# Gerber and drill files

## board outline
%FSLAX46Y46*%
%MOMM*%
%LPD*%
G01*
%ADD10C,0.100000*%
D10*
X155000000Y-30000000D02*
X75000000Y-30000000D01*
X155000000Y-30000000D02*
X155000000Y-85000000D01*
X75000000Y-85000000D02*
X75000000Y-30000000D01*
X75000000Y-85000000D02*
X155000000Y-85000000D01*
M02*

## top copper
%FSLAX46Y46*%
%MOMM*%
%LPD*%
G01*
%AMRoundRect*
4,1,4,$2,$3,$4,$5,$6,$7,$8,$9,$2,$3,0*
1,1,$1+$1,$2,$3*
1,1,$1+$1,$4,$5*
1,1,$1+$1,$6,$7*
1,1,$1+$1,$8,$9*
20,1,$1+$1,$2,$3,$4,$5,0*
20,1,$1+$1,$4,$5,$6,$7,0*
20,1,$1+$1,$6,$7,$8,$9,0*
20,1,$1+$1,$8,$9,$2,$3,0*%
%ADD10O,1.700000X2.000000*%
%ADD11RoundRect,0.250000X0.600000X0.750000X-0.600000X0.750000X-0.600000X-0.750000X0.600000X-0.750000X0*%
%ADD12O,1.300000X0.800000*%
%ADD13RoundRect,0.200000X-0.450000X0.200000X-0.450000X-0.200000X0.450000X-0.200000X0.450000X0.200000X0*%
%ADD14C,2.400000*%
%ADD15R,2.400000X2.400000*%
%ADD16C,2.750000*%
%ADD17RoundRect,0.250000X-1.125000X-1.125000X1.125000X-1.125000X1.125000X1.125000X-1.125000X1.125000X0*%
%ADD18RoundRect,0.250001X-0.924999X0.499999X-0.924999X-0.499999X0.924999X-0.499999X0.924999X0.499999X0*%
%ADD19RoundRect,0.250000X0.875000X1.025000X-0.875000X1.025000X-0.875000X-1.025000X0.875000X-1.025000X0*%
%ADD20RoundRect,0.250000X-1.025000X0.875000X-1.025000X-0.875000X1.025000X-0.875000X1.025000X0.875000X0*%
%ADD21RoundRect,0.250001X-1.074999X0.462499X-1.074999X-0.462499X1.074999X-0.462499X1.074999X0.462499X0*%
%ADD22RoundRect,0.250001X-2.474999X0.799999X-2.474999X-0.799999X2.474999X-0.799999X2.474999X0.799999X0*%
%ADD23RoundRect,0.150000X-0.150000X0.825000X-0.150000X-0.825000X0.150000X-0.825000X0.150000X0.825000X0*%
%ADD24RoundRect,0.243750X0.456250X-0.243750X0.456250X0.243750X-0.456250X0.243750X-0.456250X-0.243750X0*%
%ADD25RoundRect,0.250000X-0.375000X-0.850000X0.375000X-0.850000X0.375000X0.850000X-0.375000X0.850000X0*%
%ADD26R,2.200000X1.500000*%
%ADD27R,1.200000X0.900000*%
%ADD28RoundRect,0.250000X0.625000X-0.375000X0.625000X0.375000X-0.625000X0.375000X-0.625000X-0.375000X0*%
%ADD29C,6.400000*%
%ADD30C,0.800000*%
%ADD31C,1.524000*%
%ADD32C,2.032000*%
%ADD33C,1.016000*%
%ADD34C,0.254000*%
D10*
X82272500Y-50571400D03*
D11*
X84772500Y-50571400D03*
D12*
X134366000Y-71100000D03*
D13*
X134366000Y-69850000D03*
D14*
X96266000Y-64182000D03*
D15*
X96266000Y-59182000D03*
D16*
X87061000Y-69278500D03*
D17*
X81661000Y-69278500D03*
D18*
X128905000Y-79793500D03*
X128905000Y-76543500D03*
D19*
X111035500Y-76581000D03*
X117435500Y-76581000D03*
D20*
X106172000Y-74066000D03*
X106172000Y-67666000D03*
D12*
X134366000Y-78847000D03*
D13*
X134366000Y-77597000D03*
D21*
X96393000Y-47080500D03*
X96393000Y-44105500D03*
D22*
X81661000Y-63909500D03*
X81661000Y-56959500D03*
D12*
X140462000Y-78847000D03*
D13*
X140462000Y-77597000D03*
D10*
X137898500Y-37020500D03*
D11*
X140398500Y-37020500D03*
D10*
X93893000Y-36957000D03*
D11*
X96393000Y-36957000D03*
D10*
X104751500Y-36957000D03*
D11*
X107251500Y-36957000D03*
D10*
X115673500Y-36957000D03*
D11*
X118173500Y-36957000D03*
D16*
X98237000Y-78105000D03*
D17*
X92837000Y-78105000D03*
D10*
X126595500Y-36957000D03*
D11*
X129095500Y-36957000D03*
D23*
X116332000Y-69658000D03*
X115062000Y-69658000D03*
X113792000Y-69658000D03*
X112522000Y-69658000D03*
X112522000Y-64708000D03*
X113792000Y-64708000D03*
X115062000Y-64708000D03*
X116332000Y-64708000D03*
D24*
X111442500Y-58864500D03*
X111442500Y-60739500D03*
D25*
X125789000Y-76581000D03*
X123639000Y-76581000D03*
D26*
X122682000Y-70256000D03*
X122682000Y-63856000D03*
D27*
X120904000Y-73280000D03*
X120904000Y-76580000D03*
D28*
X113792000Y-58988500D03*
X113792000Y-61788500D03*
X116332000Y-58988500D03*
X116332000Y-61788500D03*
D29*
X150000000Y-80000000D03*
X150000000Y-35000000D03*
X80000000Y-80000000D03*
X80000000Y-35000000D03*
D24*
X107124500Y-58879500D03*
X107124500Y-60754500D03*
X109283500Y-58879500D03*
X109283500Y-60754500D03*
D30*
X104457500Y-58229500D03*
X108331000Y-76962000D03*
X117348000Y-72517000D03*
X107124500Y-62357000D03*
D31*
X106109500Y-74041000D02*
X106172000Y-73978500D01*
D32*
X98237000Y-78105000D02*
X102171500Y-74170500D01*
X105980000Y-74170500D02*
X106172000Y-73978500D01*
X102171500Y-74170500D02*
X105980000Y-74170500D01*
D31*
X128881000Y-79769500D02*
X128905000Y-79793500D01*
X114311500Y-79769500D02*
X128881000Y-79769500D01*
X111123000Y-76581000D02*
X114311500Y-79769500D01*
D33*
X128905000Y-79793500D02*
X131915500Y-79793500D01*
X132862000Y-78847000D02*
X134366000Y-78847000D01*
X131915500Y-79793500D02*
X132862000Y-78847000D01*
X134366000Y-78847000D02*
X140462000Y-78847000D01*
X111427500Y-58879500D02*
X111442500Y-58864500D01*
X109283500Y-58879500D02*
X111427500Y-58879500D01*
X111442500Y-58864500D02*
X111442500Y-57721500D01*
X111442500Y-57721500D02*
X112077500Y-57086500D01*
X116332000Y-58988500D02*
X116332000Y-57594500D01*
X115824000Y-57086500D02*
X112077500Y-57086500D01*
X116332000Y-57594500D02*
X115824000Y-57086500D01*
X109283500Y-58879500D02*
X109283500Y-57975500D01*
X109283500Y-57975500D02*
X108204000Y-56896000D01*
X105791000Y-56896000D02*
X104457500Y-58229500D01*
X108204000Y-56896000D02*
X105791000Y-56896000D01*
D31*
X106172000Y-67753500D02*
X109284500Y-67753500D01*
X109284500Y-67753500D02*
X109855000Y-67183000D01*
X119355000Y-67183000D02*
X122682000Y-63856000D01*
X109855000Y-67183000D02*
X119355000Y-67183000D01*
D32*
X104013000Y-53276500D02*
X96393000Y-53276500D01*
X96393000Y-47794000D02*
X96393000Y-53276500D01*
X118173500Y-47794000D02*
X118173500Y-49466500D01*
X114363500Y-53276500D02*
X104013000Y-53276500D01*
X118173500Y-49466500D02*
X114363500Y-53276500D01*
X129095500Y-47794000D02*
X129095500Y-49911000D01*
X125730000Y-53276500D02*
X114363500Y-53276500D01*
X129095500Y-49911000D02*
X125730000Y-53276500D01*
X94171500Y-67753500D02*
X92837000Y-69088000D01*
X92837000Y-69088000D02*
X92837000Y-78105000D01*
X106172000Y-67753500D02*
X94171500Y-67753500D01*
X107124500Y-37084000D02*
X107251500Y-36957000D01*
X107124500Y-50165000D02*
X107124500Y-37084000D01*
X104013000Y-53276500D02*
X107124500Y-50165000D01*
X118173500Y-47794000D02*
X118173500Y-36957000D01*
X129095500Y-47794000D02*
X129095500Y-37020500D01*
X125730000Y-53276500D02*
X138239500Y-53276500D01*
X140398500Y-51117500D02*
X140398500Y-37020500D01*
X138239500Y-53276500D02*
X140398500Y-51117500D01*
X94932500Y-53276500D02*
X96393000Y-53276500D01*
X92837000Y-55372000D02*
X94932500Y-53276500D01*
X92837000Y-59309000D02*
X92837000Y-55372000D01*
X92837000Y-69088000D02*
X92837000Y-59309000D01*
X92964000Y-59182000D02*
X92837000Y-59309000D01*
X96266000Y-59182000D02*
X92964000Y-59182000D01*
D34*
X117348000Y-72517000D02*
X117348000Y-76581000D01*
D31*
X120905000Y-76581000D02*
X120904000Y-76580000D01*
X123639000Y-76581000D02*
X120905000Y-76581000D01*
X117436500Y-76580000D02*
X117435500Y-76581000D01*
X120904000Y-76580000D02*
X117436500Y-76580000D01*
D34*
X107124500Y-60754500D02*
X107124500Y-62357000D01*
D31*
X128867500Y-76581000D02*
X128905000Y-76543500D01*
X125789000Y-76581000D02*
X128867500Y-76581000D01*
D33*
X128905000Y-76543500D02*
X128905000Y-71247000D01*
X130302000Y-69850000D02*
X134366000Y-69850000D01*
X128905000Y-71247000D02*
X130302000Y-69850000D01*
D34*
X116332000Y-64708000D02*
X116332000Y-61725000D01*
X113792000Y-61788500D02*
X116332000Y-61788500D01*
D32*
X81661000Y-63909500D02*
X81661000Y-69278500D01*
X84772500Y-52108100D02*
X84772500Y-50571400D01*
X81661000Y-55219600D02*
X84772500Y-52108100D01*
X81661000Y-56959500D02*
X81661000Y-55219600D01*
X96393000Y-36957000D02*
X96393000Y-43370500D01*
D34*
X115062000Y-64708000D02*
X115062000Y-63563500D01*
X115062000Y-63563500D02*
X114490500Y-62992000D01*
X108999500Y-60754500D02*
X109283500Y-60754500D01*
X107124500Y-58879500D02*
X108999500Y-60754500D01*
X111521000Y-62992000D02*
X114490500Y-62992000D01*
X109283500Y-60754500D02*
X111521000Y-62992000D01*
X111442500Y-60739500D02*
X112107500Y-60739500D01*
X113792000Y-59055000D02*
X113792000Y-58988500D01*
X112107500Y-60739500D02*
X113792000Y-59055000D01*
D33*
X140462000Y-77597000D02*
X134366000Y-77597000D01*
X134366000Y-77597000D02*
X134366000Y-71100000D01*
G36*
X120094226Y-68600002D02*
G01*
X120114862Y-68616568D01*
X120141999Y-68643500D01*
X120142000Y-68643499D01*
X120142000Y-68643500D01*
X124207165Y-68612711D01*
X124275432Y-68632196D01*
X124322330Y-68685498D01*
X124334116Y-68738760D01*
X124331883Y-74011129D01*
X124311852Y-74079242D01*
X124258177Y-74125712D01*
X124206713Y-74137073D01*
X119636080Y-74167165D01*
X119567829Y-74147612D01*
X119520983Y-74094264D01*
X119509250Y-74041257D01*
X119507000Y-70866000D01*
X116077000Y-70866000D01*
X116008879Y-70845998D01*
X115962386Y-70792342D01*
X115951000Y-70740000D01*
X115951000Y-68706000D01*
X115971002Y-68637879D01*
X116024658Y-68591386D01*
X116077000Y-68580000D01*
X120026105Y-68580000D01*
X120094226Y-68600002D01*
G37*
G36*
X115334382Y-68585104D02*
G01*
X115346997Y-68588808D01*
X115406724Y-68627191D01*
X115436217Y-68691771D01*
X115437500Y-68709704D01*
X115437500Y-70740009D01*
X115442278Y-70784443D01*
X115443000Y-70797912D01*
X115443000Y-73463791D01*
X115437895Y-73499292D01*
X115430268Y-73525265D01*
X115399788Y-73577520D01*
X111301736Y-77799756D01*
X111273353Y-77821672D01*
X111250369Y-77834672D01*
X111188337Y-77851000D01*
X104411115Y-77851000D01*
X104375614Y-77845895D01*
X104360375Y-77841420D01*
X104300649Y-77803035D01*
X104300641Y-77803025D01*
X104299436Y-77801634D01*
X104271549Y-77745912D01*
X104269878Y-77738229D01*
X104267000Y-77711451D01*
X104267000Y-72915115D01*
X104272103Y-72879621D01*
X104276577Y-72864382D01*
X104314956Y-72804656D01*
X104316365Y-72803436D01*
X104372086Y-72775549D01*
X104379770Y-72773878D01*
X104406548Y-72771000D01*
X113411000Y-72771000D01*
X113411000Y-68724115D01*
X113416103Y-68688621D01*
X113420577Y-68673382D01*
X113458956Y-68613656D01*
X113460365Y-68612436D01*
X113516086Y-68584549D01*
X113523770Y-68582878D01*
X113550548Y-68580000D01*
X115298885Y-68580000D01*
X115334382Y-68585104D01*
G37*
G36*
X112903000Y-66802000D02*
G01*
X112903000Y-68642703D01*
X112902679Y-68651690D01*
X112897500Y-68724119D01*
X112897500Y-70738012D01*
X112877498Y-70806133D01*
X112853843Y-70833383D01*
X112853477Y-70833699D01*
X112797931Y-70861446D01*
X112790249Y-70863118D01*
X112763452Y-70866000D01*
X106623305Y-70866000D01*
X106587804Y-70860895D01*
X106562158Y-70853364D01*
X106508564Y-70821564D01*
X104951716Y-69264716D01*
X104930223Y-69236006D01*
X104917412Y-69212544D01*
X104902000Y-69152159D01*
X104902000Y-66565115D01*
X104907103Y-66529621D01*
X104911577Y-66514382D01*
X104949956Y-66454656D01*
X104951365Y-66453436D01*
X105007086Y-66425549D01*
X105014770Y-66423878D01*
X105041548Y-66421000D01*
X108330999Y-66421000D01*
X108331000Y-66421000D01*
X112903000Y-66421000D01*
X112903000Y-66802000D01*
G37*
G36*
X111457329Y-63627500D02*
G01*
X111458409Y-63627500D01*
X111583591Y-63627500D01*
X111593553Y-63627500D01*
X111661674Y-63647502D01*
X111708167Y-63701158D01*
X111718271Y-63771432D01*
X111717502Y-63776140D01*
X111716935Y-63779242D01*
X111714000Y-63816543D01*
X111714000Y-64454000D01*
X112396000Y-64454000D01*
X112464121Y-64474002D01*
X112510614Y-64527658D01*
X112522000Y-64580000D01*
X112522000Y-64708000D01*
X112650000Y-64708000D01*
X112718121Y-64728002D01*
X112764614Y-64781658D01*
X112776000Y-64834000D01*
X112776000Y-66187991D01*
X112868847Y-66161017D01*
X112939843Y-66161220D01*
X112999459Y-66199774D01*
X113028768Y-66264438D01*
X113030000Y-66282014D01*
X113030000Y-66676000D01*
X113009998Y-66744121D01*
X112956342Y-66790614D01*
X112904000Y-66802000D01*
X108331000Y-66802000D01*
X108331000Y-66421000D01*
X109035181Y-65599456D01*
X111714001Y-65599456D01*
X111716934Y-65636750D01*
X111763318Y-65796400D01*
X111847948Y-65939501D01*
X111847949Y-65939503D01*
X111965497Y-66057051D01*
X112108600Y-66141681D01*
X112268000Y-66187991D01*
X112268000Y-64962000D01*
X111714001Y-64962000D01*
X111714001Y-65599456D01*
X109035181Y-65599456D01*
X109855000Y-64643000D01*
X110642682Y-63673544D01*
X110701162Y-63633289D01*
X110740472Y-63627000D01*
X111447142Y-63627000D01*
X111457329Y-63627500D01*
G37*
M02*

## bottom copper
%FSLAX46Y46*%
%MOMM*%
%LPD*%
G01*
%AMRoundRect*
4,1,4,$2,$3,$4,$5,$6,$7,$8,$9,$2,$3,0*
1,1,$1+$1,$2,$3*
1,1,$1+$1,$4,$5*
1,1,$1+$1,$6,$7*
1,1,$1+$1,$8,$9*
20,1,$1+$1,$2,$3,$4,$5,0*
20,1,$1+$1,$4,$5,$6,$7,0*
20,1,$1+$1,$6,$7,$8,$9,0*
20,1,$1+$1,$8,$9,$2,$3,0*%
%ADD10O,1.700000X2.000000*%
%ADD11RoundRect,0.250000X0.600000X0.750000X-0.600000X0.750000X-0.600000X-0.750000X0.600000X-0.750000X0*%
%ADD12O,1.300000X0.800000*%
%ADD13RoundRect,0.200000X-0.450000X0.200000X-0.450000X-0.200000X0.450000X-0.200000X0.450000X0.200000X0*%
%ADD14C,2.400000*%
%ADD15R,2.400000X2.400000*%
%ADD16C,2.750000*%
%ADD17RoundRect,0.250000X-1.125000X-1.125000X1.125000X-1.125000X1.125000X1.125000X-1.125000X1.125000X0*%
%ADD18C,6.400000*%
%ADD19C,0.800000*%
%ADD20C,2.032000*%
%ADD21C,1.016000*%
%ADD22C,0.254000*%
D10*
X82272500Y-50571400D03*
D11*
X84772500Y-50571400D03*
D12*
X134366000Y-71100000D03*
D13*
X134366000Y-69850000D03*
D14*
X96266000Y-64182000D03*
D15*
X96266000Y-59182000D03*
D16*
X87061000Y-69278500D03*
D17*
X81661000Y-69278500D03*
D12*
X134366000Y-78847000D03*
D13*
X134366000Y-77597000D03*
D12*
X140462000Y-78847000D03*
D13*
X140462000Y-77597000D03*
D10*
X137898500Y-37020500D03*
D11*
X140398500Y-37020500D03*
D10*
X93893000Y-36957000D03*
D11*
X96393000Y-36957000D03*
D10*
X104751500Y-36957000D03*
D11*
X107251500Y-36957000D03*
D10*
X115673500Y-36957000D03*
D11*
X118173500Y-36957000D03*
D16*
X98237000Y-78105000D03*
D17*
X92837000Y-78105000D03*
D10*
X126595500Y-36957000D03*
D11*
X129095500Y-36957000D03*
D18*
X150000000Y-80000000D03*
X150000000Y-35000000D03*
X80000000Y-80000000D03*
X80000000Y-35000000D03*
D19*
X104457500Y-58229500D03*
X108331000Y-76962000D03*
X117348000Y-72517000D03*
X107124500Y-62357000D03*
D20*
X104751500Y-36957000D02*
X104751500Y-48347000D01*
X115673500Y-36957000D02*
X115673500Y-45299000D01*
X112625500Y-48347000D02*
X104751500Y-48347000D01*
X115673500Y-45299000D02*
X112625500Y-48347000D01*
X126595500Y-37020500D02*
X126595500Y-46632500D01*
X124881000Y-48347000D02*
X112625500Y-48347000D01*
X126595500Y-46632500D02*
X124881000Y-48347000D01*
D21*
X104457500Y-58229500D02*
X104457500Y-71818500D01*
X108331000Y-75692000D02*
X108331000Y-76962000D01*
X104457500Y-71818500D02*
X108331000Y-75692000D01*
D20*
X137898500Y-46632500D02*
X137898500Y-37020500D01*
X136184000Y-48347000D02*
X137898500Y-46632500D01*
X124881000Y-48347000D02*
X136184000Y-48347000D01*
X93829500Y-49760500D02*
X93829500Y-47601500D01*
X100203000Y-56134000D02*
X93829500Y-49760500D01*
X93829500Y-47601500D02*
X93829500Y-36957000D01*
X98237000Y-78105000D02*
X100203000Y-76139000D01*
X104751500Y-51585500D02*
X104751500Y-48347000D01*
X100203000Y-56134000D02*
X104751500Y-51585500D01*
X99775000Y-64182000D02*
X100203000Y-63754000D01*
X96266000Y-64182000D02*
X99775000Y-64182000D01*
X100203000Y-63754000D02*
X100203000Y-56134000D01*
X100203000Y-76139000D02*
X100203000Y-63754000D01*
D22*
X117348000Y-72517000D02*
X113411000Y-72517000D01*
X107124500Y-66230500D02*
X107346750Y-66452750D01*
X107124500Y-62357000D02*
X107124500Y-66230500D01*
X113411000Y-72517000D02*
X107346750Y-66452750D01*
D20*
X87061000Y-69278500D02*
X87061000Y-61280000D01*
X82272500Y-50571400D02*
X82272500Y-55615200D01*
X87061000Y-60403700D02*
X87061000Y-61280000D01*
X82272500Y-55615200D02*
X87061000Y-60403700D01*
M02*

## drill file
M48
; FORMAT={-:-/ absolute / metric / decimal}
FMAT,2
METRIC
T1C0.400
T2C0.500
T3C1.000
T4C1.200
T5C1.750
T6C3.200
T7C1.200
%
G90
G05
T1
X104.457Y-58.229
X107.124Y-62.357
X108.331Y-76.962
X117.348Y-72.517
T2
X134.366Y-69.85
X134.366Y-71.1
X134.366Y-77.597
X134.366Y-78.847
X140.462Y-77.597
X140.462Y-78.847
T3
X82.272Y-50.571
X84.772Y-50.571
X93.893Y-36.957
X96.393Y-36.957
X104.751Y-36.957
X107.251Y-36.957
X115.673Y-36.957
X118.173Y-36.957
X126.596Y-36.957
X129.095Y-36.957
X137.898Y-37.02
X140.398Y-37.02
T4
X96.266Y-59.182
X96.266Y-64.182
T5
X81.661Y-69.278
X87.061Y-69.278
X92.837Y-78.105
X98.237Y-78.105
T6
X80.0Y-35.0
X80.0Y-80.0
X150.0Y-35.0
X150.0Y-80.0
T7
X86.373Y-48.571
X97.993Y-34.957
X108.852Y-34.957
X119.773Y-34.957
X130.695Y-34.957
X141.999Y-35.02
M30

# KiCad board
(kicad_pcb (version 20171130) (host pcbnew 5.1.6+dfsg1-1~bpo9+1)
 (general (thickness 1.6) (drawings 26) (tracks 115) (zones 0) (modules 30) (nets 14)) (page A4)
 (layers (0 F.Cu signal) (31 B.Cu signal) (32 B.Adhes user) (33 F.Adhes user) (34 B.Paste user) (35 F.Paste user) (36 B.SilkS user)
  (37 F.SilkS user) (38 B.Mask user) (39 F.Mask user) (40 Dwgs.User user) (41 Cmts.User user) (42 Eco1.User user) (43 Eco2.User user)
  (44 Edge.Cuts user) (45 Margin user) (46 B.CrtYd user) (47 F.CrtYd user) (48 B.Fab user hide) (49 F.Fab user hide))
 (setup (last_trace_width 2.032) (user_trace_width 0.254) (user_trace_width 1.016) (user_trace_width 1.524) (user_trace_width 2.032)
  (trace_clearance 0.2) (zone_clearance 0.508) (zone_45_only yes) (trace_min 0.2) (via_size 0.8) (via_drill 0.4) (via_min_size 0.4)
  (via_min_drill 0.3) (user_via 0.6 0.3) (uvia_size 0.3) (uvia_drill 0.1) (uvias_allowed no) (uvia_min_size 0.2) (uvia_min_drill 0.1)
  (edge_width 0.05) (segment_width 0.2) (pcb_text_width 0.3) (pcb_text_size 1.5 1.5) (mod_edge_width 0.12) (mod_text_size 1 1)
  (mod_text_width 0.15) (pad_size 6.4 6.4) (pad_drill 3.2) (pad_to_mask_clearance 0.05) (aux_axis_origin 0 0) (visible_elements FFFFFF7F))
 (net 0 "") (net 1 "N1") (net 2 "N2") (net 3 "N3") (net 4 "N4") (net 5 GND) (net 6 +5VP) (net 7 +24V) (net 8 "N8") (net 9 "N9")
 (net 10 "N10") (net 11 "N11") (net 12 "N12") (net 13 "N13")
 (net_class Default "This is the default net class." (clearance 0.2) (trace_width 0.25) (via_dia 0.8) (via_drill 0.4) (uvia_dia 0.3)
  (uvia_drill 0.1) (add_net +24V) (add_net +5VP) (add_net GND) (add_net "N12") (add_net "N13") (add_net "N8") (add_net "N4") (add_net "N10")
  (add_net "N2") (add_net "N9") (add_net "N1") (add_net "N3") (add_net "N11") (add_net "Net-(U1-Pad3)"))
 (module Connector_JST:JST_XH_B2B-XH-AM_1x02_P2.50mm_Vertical (layer F.Cu) (at 84.7725 50.5714 180)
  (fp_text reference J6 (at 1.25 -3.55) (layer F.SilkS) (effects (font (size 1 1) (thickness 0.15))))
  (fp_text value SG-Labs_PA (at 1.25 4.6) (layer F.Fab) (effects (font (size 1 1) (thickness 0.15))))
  (pad "" np_thru_hole circle (at -1.6 2 180) (size 1.2 1.2) (drill 1.2) (layers *.Cu *.Mask))
  (pad 2 thru_hole oval (at 2.5 0 180) (size 1.7 2) (drill 1) (layers *.Cu *.Mask) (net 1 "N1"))
  (pad 1 thru_hole roundrect (at 0 0 180) (size 1.7 2) (drill 1) (layers *.Cu *.Mask) (roundrect_rratio 0.147059) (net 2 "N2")))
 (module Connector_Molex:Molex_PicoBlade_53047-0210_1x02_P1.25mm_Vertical (layer F.Cu) (at 134.366 69.85 270)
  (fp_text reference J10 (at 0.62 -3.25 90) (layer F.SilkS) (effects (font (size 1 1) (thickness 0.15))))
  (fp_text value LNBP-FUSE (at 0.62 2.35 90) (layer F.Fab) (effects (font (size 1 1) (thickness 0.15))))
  (pad 2 thru_hole oval (at 1.25 0 270) (size 0.8 1.3) (drill 0.5) (layers *.Cu *.Mask) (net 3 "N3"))
  (pad 1 thru_hole roundrect (at 0 0 270) (size 0.8 1.3) (drill 0.5) (layers *.Cu *.Mask) (roundrect_rratio 0.25) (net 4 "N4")))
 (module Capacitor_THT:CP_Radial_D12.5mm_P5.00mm (layer F.Cu) (at 96.266 59.182 270)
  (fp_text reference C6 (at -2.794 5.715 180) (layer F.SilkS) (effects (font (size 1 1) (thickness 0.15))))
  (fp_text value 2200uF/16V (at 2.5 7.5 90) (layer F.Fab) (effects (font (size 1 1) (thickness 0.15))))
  (pad 2 thru_hole circle (at 5 0 270) (size 2.4 2.4) (drill 1.2) (layers *.Cu *.Mask) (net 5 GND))
  (pad 1 thru_hole rect (at 0 0 270) (size 2.4 2.4) (drill 1.2) (layers *.Cu *.Mask) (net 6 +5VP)))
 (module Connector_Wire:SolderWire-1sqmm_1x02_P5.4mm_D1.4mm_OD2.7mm (layer F.Cu) (at 81.661 69.2785)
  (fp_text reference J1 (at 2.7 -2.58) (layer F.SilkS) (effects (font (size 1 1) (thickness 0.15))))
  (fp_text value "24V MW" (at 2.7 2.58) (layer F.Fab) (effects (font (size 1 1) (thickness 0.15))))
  (pad 2 thru_hole circle (at 5.4 0) (size 2.75 2.75) (drill 1.75) (layers *.Cu *.Mask) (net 1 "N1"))
  (pad 1 thru_hole roundrect (at 0 0) (size 2.75 2.75) (drill 1.75) (layers *.Cu *.Mask) (roundrect_rratio 0.090909) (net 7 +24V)))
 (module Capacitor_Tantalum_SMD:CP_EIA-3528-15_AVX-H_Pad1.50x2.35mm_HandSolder (layer F.Cu) (at 128.905 78.1685 270)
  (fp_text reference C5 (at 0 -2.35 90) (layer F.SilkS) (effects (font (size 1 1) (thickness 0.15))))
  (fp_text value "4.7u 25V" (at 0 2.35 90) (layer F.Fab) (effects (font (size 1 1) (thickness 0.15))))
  (pad 2 smd roundrect (at 1.625 0 270) (size 1.5 2.35) (layers F.Cu F.Paste F.Mask) (roundrect_rratio 0.166667) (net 5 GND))
  (pad 1 smd roundrect (at -1.625 0 270) (size 1.5 2.35) (layers F.Cu F.Paste F.Mask) (roundrect_rratio 0.166667) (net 4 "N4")))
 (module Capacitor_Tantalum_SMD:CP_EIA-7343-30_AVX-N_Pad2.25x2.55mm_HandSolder (layer F.Cu) (at 114.2355 76.581 180)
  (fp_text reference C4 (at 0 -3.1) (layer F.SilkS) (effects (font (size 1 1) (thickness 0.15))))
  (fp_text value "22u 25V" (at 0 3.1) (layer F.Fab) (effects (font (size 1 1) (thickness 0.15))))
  (pad 2 smd roundrect (at 3.2 0 180) (size 2.25 2.55) (layers F.Cu F.Paste F.Mask) (roundrect_rratio 0.111111) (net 5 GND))
  (pad 1 smd roundrect (at -3.2 0 180) (size 2.25 2.55) (layers F.Cu F.Paste F.Mask) (roundrect_rratio 0.111111) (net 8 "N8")))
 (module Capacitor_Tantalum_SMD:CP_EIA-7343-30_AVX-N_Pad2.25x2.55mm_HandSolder (layer F.Cu) (at 106.172 70.866 270)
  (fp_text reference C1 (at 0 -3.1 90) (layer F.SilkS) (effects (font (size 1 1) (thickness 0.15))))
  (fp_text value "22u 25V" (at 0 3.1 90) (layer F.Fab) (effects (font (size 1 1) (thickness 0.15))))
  (pad 2 smd roundrect (at 3.2 0 270) (size 2.25 2.55) (layers F.Cu F.Paste F.Mask) (roundrect_rratio 0.111111) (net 5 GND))
  (pad 1 smd roundrect (at -3.2 0 270) (size 2.25 2.55) (layers F.Cu F.Paste F.Mask) (roundrect_rratio 0.111111) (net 6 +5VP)))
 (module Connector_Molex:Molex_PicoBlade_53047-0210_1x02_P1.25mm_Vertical (layer F.Cu) (at 134.366 77.597 270)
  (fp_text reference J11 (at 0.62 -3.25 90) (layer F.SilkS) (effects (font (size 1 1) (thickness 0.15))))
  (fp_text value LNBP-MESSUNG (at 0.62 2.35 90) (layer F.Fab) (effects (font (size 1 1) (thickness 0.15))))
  (pad 2 thru_hole oval (at 1.25 0 270) (size 0.8 1.3) (drill 0.5) (layers *.Cu *.Mask) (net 5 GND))
  (pad 1 thru_hole roundrect (at 0 0 270) (size 0.8 1.3) (drill 0.5) (layers *.Cu *.Mask) (roundrect_rratio 0.25) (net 3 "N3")))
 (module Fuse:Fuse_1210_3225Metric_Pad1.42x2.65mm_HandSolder (layer F.Cu) (at 96.393 45.593 270)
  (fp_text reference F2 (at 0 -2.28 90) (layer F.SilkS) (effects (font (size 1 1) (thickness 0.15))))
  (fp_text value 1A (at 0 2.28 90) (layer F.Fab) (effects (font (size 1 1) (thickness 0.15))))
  (pad 2 smd roundrect (at 1.4875 0 270) (size 1.425 2.65) (layers F.Cu F.Paste F.Mask) (roundrect_rratio 0.175439) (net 6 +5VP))
  (pad 1 smd roundrect (at -1.4875 0 270) (size 1.425 2.65) (layers F.Cu F.Paste F.Mask) (roundrect_rratio 0.175439) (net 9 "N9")))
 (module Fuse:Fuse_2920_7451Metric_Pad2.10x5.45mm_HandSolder (layer F.Cu) (at 81.661 60.4345 270)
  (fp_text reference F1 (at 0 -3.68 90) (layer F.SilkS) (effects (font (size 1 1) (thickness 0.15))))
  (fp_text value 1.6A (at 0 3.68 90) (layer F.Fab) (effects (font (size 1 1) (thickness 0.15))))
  (pad 2 smd roundrect (at 3.475 0 270) (size 2.1 5.45) (layers F.Cu F.Paste F.Mask) (roundrect_rratio 0.119048) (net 7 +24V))
  (pad 1 smd roundrect (at -3.475 0 270) (size 2.1 5.45) (layers F.Cu F.Paste F.Mask) (roundrect_rratio 0.119048) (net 2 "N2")))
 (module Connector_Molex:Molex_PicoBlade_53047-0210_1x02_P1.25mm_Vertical (layer F.Cu) (at 140.462 77.597 270)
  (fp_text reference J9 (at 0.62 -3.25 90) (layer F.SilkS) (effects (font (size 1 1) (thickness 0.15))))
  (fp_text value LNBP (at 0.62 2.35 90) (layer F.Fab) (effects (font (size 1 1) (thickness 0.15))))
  (pad 2 thru_hole oval (at 1.25 0 270) (size 0.8 1.3) (drill 0.5) (layers *.Cu *.Mask) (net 5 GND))
  (pad 1 thru_hole roundrect (at 0 0 270) (size 0.8 1.3) (drill 0.5) (layers *.Cu *.Mask) (roundrect_rratio 0.25) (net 3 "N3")))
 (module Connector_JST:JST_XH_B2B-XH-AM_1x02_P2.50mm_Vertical (layer F.Cu) (at 140.3985 37.0205 180)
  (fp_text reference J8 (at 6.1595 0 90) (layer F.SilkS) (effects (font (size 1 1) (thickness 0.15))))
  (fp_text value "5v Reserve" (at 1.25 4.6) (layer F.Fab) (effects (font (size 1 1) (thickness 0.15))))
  (pad "" np_thru_hole circle (at -1.6 2 180) (size 1.2 1.2) (drill 1.2) (layers *.Cu *.Mask))
  (pad 2 thru_hole oval (at 2.5 0 180) (size 1.7 2) (drill 1) (layers *.Cu *.Mask) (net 5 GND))
  (pad 1 thru_hole roundrect (at 0 0 180) (size 1.7 2) (drill 1) (layers *.Cu *.Mask) (roundrect_rratio 0.147059) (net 6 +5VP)))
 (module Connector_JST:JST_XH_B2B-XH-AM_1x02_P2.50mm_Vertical (layer F.Cu) (at 96.393 36.957 180)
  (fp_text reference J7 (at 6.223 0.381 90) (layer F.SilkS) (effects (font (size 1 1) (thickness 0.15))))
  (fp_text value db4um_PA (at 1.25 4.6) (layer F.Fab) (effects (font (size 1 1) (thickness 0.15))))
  (pad "" np_thru_hole circle (at -1.6 2 180) (size 1.2 1.2) (drill 1.2) (layers *.Cu *.Mask))
  (pad 2 thru_hole oval (at 2.5 0 180) (size 1.7 2) (drill 1) (layers *.Cu *.Mask) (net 5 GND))
  (pad 1 thru_hole roundrect (at 0 0 180) (size 1.7 2) (drill 1) (layers *.Cu *.Mask) (roundrect_rratio 0.147059) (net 9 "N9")))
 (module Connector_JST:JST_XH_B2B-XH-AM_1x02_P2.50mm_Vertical (layer F.Cu) (at 107.2515 36.957 180)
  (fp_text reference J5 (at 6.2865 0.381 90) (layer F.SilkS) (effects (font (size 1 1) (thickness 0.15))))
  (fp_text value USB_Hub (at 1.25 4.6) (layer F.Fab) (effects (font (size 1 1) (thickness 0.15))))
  (pad "" np_thru_hole circle (at -1.6 2 180) (size 1.2 1.2) (drill 1.2) (layers *.Cu *.Mask))
  (pad 2 thru_hole oval (at 2.5 0 180) (size 1.7 2) (drill 1) (layers *.Cu *.Mask) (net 5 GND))
  (pad 1 thru_hole roundrect (at 0 0 180) (size 1.7 2) (drill 1) (layers *.Cu *.Mask) (roundrect_rratio 0.147059) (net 6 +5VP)))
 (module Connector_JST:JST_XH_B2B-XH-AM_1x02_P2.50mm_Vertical (layer F.Cu) (at 118.1735 36.957 180)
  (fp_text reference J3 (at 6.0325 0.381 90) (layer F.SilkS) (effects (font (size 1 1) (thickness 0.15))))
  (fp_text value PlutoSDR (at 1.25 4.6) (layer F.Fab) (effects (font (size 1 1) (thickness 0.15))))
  (pad "" np_thru_hole circle (at -1.6 2 180) (size 1.2 1.2) (drill 1.2) (layers *.Cu *.Mask))
  (pad 2 thru_hole oval (at 2.5 0 180) (size 1.7 2) (drill 1) (layers *.Cu *.Mask) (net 5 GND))
  (pad 1 thru_hole roundrect (at 0 0 180) (size 1.7 2) (drill 1) (layers *.Cu *.Mask) (roundrect_rratio 0.147059) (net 6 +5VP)))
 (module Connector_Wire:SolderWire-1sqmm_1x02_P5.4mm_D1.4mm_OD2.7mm (layer F.Cu) (at 92.837 78.105)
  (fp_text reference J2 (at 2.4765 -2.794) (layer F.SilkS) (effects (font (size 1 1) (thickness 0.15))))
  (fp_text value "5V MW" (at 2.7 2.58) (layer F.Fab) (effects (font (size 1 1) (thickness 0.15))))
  (pad 2 thru_hole circle (at 5.4 0) (size 2.75 2.75) (drill 1.75) (layers *.Cu *.Mask) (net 5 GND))
  (pad 1 thru_hole roundrect (at 0 0) (size 2.75 2.75) (drill 1.75) (layers *.Cu *.Mask) (roundrect_rratio 0.090909) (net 6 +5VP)))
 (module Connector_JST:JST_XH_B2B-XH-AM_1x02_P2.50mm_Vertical (layer F.Cu) (at 129.0955 36.957 180)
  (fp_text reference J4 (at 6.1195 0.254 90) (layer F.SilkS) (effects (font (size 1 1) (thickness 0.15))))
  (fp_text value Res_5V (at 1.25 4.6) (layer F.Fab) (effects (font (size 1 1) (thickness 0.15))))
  (pad "" np_thru_hole circle (at -1.6 2 180) (size 1.2 1.2) (drill 1.2) (layers *.Cu *.Mask))
  (pad 2 thru_hole oval (at 2.5 0 180) (size 1.7 2) (drill 1) (layers *.Cu *.Mask) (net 5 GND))
  (pad 1 thru_hole roundrect (at 0 0 180) (size 1.7 2) (drill 1) (layers *.Cu *.Mask) (roundrect_rratio 0.147059) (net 6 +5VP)))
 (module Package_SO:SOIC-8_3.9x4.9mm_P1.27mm (layer F.Cu) (at 114.427 67.183 270)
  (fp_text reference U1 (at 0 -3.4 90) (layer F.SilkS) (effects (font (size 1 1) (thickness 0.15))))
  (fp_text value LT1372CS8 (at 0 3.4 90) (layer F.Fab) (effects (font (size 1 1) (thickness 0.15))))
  (pad 8 smd roundrect (at 2.475 -1.905 270) (size 1.95 0.6) (layers F.Cu F.Paste F.Mask) (roundrect_rratio 0.25) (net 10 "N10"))
  (pad 7 smd roundrect (at 2.475 -0.635 270) (size 1.95 0.6) (layers F.Cu F.Paste F.Mask) (roundrect_rratio 0.25) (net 5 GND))
  (pad 6 smd roundrect (at 2.475 0.635 270) (size 1.95 0.6) (layers F.Cu F.Paste F.Mask) (roundrect_rratio 0.25) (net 5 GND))
  (pad 5 smd roundrect (at 2.475 1.905 270) (size 1.95 0.6) (layers F.Cu F.Paste F.Mask) (roundrect_rratio 0.25) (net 6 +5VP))
  (pad 4 smd roundrect (at -2.475 1.905 270) (size 1.95 0.6) (layers F.Cu F.Paste F.Mask) (roundrect_rratio 0.25) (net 6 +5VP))
  (pad 3 smd roundrect (at -2.475 0.635 270) (size 1.95 0.6) (layers F.Cu F.Paste F.Mask) (roundrect_rratio 0.25))
  (pad 2 smd roundrect (at -2.475 -0.635 270) (size 1.95 0.6) (layers F.Cu F.Paste F.Mask) (roundrect_rratio 0.25) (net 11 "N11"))
  (pad 1 smd roundrect (at -2.475 -1.905 270) (size 1.95 0.6) (layers F.Cu F.Paste F.Mask) (roundrect_rratio 0.25) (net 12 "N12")))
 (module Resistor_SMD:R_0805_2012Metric (layer F.Cu) (at 111.4425 59.802 90)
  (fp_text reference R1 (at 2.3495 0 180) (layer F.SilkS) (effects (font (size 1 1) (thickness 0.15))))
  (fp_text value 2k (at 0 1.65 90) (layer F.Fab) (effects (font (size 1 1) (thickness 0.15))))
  (pad 2 smd roundrect (at 0.9375 0 90) (size 0.975 1.4) (layers F.Cu F.Paste F.Mask) (roundrect_rratio 0.25) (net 5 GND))
  (pad 1 smd roundrect (at -0.9375 0 90) (size 0.975 1.4) (layers F.Cu F.Paste F.Mask) (roundrect_rratio 0.25) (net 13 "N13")))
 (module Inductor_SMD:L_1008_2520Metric (layer F.Cu) (at 124.714 76.581)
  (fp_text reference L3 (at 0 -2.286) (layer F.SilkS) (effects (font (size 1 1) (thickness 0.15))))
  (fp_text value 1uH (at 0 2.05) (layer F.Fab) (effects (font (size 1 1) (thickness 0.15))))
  (pad 2 smd roundrect (at 1.075 0) (size 1.25 2.2) (layers F.Cu F.Paste F.Mask) (roundrect_rratio 0.2) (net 4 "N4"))
  (pad 1 smd roundrect (at -1.075 0) (size 1.25 2.2) (layers F.Cu F.Paste F.Mask) (roundrect_rratio 0.2) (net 8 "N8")))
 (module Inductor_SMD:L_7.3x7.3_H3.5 (layer F.Cu) (at 122.682 67.056 270)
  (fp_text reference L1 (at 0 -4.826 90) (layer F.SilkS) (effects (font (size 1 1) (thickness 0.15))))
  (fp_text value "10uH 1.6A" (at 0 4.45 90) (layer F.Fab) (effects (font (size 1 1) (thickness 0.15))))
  (pad 2 smd rect (at 3.2 0 270) (size 1.5 2.2) (layers F.Cu F.Paste F.Mask) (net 10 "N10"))
  (pad 1 smd rect (at -3.2 0 270) (size 1.5 2.2) (layers F.Cu F.Paste F.Mask) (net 6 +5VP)))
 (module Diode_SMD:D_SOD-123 (layer F.Cu) (at 120.904 74.93 90)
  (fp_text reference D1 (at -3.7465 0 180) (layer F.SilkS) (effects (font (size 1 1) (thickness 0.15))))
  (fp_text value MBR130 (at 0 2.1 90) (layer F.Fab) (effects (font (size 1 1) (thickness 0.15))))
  (pad 2 smd rect (at 1.65 0 90) (size 0.9 1.2) (layers F.Cu F.Paste F.Mask) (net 10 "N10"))
  (pad 1 smd rect (at -1.65 0 90) (size 0.9 1.2) (layers F.Cu F.Paste F.Mask) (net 8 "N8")))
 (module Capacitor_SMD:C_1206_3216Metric (layer F.Cu) (at 113.792 60.3885 90)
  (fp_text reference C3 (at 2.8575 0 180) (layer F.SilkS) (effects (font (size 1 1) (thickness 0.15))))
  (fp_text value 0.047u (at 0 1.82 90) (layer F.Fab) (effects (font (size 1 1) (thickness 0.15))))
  (pad 2 smd roundrect (at 1.4 0 90) (size 1.25 1.75) (layers F.Cu F.Paste F.Mask) (roundrect_rratio 0.2) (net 13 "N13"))
  (pad 1 smd roundrect (at -1.4 0 90) (size 1.25 1.75) (layers F.Cu F.Paste F.Mask) (roundrect_rratio 0.2) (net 12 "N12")))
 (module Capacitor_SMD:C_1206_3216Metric (layer F.Cu) (at 116.332 60.3885 90)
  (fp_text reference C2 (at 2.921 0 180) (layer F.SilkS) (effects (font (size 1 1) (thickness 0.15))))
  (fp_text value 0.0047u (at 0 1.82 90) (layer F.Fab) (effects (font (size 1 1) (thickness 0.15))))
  (pad 2 smd roundrect (at 1.4 0 90) (size 1.25 1.75) (layers F.Cu F.Paste F.Mask) (roundrect_rratio 0.2) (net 5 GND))
  (pad 1 smd roundrect (at -1.4 0 90) (size 1.25 1.75) (layers F.Cu F.Paste F.Mask) (roundrect_rratio 0.2) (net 12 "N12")))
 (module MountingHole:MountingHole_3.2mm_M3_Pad (layer F.Cu) (at 150 80)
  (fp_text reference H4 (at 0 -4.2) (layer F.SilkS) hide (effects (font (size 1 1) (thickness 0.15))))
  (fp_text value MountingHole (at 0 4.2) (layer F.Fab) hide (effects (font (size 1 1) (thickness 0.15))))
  (pad 1 thru_hole circle (at 0 0) (size 6.4 6.4) (drill 3.2) (layers *.Cu *.Mask)))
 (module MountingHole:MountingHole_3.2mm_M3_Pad (layer F.Cu) (at 150 35)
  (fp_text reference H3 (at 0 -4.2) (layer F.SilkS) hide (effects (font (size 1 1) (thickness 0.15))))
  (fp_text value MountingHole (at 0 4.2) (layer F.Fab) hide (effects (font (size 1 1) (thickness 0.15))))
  (pad 1 thru_hole circle (at 0 0) (size 6.4 6.4) (drill 3.2) (layers *.Cu *.Mask)))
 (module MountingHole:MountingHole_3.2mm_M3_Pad (layer F.Cu) (at 80 80)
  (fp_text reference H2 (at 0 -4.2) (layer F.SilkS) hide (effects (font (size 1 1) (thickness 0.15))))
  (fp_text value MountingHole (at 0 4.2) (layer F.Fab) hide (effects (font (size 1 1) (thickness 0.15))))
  (pad 1 thru_hole circle (at 0 0) (size 6.4 6.4) (drill 3.2) (layers *.Cu *.Mask)))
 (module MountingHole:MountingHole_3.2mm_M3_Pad (layer F.Cu) (at 80 35)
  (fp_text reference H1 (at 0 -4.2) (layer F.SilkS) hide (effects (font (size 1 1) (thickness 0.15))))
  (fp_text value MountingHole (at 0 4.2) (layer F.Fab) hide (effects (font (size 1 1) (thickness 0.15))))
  (pad 1 thru_hole circle (at 0 0) (size 6.4 6.4) (drill 3.2) (layers *.Cu *.Mask)))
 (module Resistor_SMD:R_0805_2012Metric (layer F.Cu) (at 107.1245 59.817 90)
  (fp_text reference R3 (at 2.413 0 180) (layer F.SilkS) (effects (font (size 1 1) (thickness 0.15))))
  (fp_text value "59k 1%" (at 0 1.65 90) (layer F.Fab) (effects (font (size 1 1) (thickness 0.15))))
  (pad 2 smd roundrect (at 0.9375 0 90) (size 0.975 1.4) (layers F.Cu F.Paste F.Mask) (roundrect_rratio 0.25) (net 11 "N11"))
  (pad 1 smd roundrect (at -0.9375 0 90) (size 0.975 1.4) (layers F.Cu F.Paste F.Mask) (roundrect_rratio 0.25) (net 8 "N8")))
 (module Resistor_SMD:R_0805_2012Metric (layer F.Cu) (at 109.2835 59.817 90)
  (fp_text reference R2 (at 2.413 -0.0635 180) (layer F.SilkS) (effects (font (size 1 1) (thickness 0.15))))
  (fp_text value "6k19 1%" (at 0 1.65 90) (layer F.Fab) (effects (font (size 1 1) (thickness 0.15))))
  (pad 2 smd roundrect (at 0.9375 0 90) (size 0.975 1.4) (layers F.Cu F.Paste F.Mask) (roundrect_rratio 0.25) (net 5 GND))
  (pad 1 smd roundrect (at -0.9375 0 90) (size 0.975 1.4) (layers F.Cu F.Paste F.Mask) (roundrect_rratio 0.25) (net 11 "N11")))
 (gr_line (start 155 30) (end 75 30) (layer Edge.Cuts) (width 0.1))
 (gr_line (start 155 30) (end 155 85) (layer Edge.Cuts) (width 0.1))
 (gr_line (start 75 85) (end 75 30) (layer Edge.Cuts) (width 0.1))
 (gr_line (start 75 85) (end 155 85) (layer Edge.Cuts) (width 0.1))
 (segment (start 106.1095 74.041) (end 106.172 73.9785) (width 1.524) (layer F.Cu) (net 5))
 (segment (start 104.7515 36.957) (end 104.7515 48.347) (width 2.032) (layer B.Cu) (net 5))
 (segment (start 115.6735 36.957) (end 115.6735 45.299) (width 2.032) (layer B.Cu) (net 5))
 (segment (start 112.6255 48.347) (end 104.7515 48.347) (width 2.032) (layer B.Cu) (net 5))
 (segment (start 115.6735 45.299) (end 112.6255 48.347) (width 2.032) (layer B.Cu) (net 5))
 (segment (start 126.5955 37.0205) (end 126.5955 46.6325) (width 2.032) (layer B.Cu) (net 5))
 (segment (start 124.881 48.347) (end 112.6255 48.347) (width 2.032) (layer B.Cu) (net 5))
 (segment (start 126.5955 46.6325) (end 124.881 48.347) (width 2.032) (layer B.Cu) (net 5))
 (segment (start 98.237 78.105) (end 102.1715 74.1705) (width 2.032) (layer F.Cu) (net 5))
 (segment (start 105.98 74.1705) (end 106.172 73.9785) (width 2.032) (layer F.Cu) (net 5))
 (segment (start 102.1715 74.1705) (end 105.98 74.1705) (width 2.032) (layer F.Cu) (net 5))
 (segment (start 128.881 79.7695) (end 128.905 79.7935) (width 1.524) (layer F.Cu) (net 5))
 (segment (start 114.3115 79.7695) (end 128.881 79.7695) (width 1.524) (layer F.Cu) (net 5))
 (segment (start 111.123 76.581) (end 114.3115 79.7695) (width 1.524) (layer F.Cu) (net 5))
 (segment (start 128.905 79.7935) (end 131.9155 79.7935) (width 1.016) (layer F.Cu) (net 5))
 (segment (start 132.862 78.847) (end 134.366 78.847) (width 1.016) (layer F.Cu) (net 5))
 (segment (start 131.9155 79.7935) (end 132.862 78.847) (width 1.016) (layer F.Cu) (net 5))
 (segment (start 134.366 78.847) (end 140.462 78.847) (width 1.016) (layer F.Cu) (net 5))
 (segment (start 111.4275 58.8795) (end 111.4425 58.8645) (width 1.016) (layer F.Cu) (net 5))
 (segment (start 109.2835 58.8795) (end 111.4275 58.8795) (width 1.016) (layer F.Cu) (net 5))
 (segment (start 111.4425 58.8645) (end 111.4425 57.7215) (width 1.016) (layer F.Cu) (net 5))
 (segment (start 111.4425 57.7215) (end 112.0775 57.0865) (width 1.016) (layer F.Cu) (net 5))
 (segment (start 116.332 58.9885) (end 116.332 57.5945) (width 1.016) (layer F.Cu) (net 5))
 (segment (start 115.824 57.0865) (end 112.0775 57.0865) (width 1.016) (layer F.Cu) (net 5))
 (segment (start 116.332 57.5945) (end 115.824 57.0865) (width 1.016) (layer F.Cu) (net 5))
 (segment (start 109.2835 58.8795) (end 109.2835 57.9755) (width 1.016) (layer F.Cu) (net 5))
 (segment (start 109.2835 57.9755) (end 108.204 56.896) (width 1.016) (layer F.Cu) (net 5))
 (segment (start 105.791 56.896) (end 104.4575 58.2295) (width 1.016) (layer F.Cu) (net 5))
 (via (at 104.4575 58.2295) (size 0.8) (drill 0.4) (layers F.Cu B.Cu) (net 5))
 (segment (start 108.204 56.896) (end 105.791 56.896) (width 1.016) (layer F.Cu) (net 5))
 (segment (start 104.4575 58.2295) (end 104.4575 71.8185) (width 1.016) (layer B.Cu) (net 5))
 (segment (start 108.331 75.692) (end 108.331 76.962) (width 1.016) (layer B.Cu) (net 5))
 (via (at 108.331 76.962) (size 0.8) (drill 0.4) (layers F.Cu B.Cu) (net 5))
 (segment (start 104.4575 71.8185) (end 108.331 75.692) (width 1.016) (layer B.Cu) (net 5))
 (segment (start 137.8985 46.6325) (end 137.8985 37.0205) (width 2.032) (layer B.Cu) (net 5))
 (segment (start 136.184 48.347) (end 137.8985 46.6325) (width 2.032) (layer B.Cu) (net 5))
 (segment (start 124.881 48.347) (end 136.184 48.347) (width 2.032) (layer B.Cu) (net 5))
 (segment (start 93.8295 49.7605) (end 93.8295 47.6015) (width 2.032) (layer B.Cu) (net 5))
 (segment (start 100.203 56.134) (end 93.8295 49.7605) (width 2.032) (layer B.Cu) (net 5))
 (segment (start 93.8295 47.6015) (end 93.8295 36.957) (width 2.032) (layer B.Cu) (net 5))
 (segment (start 98.237 78.105) (end 100.203 76.139) (width 2.032) (layer B.Cu) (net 5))
 (segment (start 104.7515 51.5855) (end 104.7515 48.347) (width 2.032) (layer B.Cu) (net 5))
 (segment (start 100.203 56.134) (end 104.7515 51.5855) (width 2.032) (layer B.Cu) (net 5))
 (segment (start 99.775 64.182) (end 100.203 63.754) (width 2.032) (layer B.Cu) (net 5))
 (segment (start 96.266 64.182) (end 99.775 64.182) (width 2.032) (layer B.Cu) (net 5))
 (segment (start 100.203 63.754) (end 100.203 56.134) (width 2.032) (layer B.Cu) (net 5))
 (segment (start 100.203 76.139) (end 100.203 63.754) (width 2.032) (layer B.Cu) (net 5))
 (segment (start 106.172 67.7535) (end 109.2845 67.7535) (width 1.524) (layer F.Cu) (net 6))
 (segment (start 109.2845 67.7535) (end 109.855 67.183) (width 1.524) (layer F.Cu) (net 6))
 (segment (start 119.355 67.183) (end 122.682 63.856) (width 1.524) (layer F.Cu) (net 6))
 (segment (start 109.855 67.183) (end 119.355 67.183) (width 1.524) (layer F.Cu) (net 6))
 (segment (start 104.013 53.2765) (end 96.393 53.2765) (width 2.032) (layer F.Cu) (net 6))
 (segment (start 96.393 47.794) (end 96.393 53.2765) (width 2.032) (layer F.Cu) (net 6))
 (segment (start 118.1735 47.794) (end 118.1735 49.4665) (width 2.032) (layer F.Cu) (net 6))
 (segment (start 114.3635 53.2765) (end 104.013 53.2765) (width 2.032) (layer F.Cu) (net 6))
 (segment (start 118.1735 49.4665) (end 114.3635 53.2765) (width 2.032) (layer F.Cu) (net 6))
 (segment (start 129.0955 47.794) (end 129.0955 49.911) (width 2.032) (layer F.Cu) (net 6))
 (segment (start 125.73 53.2765) (end 114.3635 53.2765) (width 2.032) (layer F.Cu) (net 6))
 (segment (start 129.0955 49.911) (end 125.73 53.2765) (width 2.032) (layer F.Cu) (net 6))
 (segment (start 94.1715 67.7535) (end 92.837 69.088) (width 2.032) (layer F.Cu) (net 6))
 (segment (start 92.837 69.088) (end 92.837 78.105) (width 2.032) (layer F.Cu) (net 6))
 (segment (start 106.172 67.7535) (end 94.1715 67.7535) (width 2.032) (layer F.Cu) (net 6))
 (segment (start 107.1245 37.084) (end 107.2515 36.957) (width 2.032) (layer F.Cu) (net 6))
 (segment (start 107.1245 50.165) (end 107.1245 37.084) (width 2.032) (layer F.Cu) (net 6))
 (segment (start 104.013 53.2765) (end 107.1245 50.165) (width 2.032) (layer F.Cu) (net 6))
 (segment (start 118.1735 47.794) (end 118.1735 36.957) (width 2.032) (layer F.Cu) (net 6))
 (segment (start 129.0955 47.794) (end 129.0955 37.0205) (width 2.032) (layer F.Cu) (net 6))
 (segment (start 125.73 53.2765) (end 138.2395 53.2765) (width 2.032) (layer F.Cu) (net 6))
 (segment (start 140.3985 51.1175) (end 140.3985 37.0205) (width 2.032) (layer F.Cu) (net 6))
 (segment (start 138.2395 53.2765) (end 140.3985 51.1175) (width 2.032) (layer F.Cu) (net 6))
 (segment (start 94.9325 53.2765) (end 96.393 53.2765) (width 2.032) (layer F.Cu) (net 6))
 (segment (start 92.837 55.372) (end 94.9325 53.2765) (width 2.032) (layer F.Cu) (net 6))
 (segment (start 92.837 59.309) (end 92.837 55.372) (width 2.032) (layer F.Cu) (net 6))
 (segment (start 92.837 69.088) (end 92.837 59.309) (width 2.032) (layer F.Cu) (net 6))
 (segment (start 92.964 59.182) (end 92.837 59.309) (width 2.032) (layer F.Cu) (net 6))
 (segment (start 96.266 59.182) (end 92.964 59.182) (width 2.032) (layer F.Cu) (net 6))
 (via (at 117.348 72.517) (size 0.8) (drill 0.4) (layers F.Cu B.Cu) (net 8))
 (segment (start 117.348 72.517) (end 117.348 76.581) (width 0.254) (layer F.Cu) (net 8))
 (segment (start 120.905 76.581) (end 120.904 76.58) (width 1.524) (layer F.Cu) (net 8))
 (segment (start 123.639 76.581) (end 120.905 76.581) (width 1.524) (layer F.Cu) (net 8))
 (segment (start 117.4365 76.58) (end 117.4355 76.581) (width 1.524) (layer F.Cu) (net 8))
 (segment (start 120.904 76.58) (end 117.4365 76.58) (width 1.524) (layer F.Cu) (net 8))
 (segment (start 117.348 72.517) (end 113.411 72.517) (width 0.254) (layer B.Cu) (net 8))
 (via (at 107.1245 62.357) (size 0.8) (drill 0.4) (layers F.Cu B.Cu) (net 8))
 (segment (start 107.1245 60.7545) (end 107.1245 62.357) (width 0.254) (layer F.Cu) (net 8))
 (segment (start 107.1245 66.2305) (end 107.34675 66.45275) (width 0.254) (layer B.Cu) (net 8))
 (segment (start 107.1245 62.357) (end 107.1245 66.2305) (width 0.254) (layer B.Cu) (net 8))
 (segment (start 113.411 72.517) (end 107.34675 66.45275) (width 0.254) (layer B.Cu) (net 8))
 (segment (start 128.8675 76.581) (end 128.905 76.5435) (width 1.524) (layer F.Cu) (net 4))
 (segment (start 125.789 76.581) (end 128.8675 76.581) (width 1.524) (layer F.Cu) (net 4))
 (segment (start 128.905 76.5435) (end 128.905 71.247) (width 1.016) (layer F.Cu) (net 4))
 (segment (start 130.302 69.85) (end 134.366 69.85) (width 1.016) (layer F.Cu) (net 4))
 (segment (start 128.905 71.247) (end 130.302 69.85) (width 1.016) (layer F.Cu) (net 4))
 (segment (start 116.332 64.708) (end 116.332 61.725) (width 0.254) (layer F.Cu) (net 12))
 (segment (start 113.792 61.7885) (end 116.332 61.7885) (width 0.254) (layer F.Cu) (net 12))
 (segment (start 81.661 63.9095) (end 81.661 69.2785) (width 2.032) (layer F.Cu) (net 7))
 (segment (start 84.7725 52.1081) (end 84.7725 50.5714) (width 2.032) (layer F.Cu) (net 2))
 (segment (start 81.661 55.2196) (end 84.7725 52.1081) (width 2.032) (layer F.Cu) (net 2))
 (segment (start 81.661 56.9595) (end 81.661 55.2196) (width 2.032) (layer F.Cu) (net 2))
 (segment (start 96.393 36.957) (end 96.393 43.3705) (width 2.032) (layer F.Cu) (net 9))
 (segment (start 115.062 64.708) (end 115.062 63.5635) (width 0.254) (layer F.Cu) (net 11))
 (segment (start 115.062 63.5635) (end 114.4905 62.992) (width 0.254) (layer F.Cu) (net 11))
 (segment (start 108.9995 60.7545) (end 109.2835 60.7545) (width 0.254) (layer F.Cu) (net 11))
 (segment (start 107.1245 58.8795) (end 108.9995 60.7545) (width 0.254) (layer F.Cu) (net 11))
 (segment (start 111.521 62.992) (end 114.4905 62.992) (width 0.254) (layer F.Cu) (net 11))
 (segment (start 109.2835 60.7545) (end 111.521 62.992) (width 0.254) (layer F.Cu) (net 11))
 (segment (start 111.4425 60.7395) (end 112.1075 60.7395) (width 0.254) (layer F.Cu) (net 13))
 (segment (start 113.792 59.055) (end 113.792 58.9885) (width 0.254) (layer F.Cu) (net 13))
 (segment (start 112.1075 60.7395) (end 113.792 59.055) (width 0.254) (layer F.Cu) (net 13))
 (segment (start 87.061 69.2785) (end 87.061 61.28) (width 2.032) (layer B.Cu) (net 1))
 (segment (start 82.2725 50.5714) (end 82.2725 55.6152) (width 2.032) (layer B.Cu) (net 1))
 (segment (start 87.061 60.4037) (end 87.061 61.28) (width 2.032) (layer B.Cu) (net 1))
 (segment (start 82.2725 55.6152) (end 87.061 60.4037) (width 2.032) (layer B.Cu) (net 1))
 (segment (start 140.462 77.597) (end 134.366 77.597) (width 1.016) (layer F.Cu) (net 3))
 (segment (start 134.366 77.597) (end 134.366 71.1) (width 1.016) (layer F.Cu) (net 3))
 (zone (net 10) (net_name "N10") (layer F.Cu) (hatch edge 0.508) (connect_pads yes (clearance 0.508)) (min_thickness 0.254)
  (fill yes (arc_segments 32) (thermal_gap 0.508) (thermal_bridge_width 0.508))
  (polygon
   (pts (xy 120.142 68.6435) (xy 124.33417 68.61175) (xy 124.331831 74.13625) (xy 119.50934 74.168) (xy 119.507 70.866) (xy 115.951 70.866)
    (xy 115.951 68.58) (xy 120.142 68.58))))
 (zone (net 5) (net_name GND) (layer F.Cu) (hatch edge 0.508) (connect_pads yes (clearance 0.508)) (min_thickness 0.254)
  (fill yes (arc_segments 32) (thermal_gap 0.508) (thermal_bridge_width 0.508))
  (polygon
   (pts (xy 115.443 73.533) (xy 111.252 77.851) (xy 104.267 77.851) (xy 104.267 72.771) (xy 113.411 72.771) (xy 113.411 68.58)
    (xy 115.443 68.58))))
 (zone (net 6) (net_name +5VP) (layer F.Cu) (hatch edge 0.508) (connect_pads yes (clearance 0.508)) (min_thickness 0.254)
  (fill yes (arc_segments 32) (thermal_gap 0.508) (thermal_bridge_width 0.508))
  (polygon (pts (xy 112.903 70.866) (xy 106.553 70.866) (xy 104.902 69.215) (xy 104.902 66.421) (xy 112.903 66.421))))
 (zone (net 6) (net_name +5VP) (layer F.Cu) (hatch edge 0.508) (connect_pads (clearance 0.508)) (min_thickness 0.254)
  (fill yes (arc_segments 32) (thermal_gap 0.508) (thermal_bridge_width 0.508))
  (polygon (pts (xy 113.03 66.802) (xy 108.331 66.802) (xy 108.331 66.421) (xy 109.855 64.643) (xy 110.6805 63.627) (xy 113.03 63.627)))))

